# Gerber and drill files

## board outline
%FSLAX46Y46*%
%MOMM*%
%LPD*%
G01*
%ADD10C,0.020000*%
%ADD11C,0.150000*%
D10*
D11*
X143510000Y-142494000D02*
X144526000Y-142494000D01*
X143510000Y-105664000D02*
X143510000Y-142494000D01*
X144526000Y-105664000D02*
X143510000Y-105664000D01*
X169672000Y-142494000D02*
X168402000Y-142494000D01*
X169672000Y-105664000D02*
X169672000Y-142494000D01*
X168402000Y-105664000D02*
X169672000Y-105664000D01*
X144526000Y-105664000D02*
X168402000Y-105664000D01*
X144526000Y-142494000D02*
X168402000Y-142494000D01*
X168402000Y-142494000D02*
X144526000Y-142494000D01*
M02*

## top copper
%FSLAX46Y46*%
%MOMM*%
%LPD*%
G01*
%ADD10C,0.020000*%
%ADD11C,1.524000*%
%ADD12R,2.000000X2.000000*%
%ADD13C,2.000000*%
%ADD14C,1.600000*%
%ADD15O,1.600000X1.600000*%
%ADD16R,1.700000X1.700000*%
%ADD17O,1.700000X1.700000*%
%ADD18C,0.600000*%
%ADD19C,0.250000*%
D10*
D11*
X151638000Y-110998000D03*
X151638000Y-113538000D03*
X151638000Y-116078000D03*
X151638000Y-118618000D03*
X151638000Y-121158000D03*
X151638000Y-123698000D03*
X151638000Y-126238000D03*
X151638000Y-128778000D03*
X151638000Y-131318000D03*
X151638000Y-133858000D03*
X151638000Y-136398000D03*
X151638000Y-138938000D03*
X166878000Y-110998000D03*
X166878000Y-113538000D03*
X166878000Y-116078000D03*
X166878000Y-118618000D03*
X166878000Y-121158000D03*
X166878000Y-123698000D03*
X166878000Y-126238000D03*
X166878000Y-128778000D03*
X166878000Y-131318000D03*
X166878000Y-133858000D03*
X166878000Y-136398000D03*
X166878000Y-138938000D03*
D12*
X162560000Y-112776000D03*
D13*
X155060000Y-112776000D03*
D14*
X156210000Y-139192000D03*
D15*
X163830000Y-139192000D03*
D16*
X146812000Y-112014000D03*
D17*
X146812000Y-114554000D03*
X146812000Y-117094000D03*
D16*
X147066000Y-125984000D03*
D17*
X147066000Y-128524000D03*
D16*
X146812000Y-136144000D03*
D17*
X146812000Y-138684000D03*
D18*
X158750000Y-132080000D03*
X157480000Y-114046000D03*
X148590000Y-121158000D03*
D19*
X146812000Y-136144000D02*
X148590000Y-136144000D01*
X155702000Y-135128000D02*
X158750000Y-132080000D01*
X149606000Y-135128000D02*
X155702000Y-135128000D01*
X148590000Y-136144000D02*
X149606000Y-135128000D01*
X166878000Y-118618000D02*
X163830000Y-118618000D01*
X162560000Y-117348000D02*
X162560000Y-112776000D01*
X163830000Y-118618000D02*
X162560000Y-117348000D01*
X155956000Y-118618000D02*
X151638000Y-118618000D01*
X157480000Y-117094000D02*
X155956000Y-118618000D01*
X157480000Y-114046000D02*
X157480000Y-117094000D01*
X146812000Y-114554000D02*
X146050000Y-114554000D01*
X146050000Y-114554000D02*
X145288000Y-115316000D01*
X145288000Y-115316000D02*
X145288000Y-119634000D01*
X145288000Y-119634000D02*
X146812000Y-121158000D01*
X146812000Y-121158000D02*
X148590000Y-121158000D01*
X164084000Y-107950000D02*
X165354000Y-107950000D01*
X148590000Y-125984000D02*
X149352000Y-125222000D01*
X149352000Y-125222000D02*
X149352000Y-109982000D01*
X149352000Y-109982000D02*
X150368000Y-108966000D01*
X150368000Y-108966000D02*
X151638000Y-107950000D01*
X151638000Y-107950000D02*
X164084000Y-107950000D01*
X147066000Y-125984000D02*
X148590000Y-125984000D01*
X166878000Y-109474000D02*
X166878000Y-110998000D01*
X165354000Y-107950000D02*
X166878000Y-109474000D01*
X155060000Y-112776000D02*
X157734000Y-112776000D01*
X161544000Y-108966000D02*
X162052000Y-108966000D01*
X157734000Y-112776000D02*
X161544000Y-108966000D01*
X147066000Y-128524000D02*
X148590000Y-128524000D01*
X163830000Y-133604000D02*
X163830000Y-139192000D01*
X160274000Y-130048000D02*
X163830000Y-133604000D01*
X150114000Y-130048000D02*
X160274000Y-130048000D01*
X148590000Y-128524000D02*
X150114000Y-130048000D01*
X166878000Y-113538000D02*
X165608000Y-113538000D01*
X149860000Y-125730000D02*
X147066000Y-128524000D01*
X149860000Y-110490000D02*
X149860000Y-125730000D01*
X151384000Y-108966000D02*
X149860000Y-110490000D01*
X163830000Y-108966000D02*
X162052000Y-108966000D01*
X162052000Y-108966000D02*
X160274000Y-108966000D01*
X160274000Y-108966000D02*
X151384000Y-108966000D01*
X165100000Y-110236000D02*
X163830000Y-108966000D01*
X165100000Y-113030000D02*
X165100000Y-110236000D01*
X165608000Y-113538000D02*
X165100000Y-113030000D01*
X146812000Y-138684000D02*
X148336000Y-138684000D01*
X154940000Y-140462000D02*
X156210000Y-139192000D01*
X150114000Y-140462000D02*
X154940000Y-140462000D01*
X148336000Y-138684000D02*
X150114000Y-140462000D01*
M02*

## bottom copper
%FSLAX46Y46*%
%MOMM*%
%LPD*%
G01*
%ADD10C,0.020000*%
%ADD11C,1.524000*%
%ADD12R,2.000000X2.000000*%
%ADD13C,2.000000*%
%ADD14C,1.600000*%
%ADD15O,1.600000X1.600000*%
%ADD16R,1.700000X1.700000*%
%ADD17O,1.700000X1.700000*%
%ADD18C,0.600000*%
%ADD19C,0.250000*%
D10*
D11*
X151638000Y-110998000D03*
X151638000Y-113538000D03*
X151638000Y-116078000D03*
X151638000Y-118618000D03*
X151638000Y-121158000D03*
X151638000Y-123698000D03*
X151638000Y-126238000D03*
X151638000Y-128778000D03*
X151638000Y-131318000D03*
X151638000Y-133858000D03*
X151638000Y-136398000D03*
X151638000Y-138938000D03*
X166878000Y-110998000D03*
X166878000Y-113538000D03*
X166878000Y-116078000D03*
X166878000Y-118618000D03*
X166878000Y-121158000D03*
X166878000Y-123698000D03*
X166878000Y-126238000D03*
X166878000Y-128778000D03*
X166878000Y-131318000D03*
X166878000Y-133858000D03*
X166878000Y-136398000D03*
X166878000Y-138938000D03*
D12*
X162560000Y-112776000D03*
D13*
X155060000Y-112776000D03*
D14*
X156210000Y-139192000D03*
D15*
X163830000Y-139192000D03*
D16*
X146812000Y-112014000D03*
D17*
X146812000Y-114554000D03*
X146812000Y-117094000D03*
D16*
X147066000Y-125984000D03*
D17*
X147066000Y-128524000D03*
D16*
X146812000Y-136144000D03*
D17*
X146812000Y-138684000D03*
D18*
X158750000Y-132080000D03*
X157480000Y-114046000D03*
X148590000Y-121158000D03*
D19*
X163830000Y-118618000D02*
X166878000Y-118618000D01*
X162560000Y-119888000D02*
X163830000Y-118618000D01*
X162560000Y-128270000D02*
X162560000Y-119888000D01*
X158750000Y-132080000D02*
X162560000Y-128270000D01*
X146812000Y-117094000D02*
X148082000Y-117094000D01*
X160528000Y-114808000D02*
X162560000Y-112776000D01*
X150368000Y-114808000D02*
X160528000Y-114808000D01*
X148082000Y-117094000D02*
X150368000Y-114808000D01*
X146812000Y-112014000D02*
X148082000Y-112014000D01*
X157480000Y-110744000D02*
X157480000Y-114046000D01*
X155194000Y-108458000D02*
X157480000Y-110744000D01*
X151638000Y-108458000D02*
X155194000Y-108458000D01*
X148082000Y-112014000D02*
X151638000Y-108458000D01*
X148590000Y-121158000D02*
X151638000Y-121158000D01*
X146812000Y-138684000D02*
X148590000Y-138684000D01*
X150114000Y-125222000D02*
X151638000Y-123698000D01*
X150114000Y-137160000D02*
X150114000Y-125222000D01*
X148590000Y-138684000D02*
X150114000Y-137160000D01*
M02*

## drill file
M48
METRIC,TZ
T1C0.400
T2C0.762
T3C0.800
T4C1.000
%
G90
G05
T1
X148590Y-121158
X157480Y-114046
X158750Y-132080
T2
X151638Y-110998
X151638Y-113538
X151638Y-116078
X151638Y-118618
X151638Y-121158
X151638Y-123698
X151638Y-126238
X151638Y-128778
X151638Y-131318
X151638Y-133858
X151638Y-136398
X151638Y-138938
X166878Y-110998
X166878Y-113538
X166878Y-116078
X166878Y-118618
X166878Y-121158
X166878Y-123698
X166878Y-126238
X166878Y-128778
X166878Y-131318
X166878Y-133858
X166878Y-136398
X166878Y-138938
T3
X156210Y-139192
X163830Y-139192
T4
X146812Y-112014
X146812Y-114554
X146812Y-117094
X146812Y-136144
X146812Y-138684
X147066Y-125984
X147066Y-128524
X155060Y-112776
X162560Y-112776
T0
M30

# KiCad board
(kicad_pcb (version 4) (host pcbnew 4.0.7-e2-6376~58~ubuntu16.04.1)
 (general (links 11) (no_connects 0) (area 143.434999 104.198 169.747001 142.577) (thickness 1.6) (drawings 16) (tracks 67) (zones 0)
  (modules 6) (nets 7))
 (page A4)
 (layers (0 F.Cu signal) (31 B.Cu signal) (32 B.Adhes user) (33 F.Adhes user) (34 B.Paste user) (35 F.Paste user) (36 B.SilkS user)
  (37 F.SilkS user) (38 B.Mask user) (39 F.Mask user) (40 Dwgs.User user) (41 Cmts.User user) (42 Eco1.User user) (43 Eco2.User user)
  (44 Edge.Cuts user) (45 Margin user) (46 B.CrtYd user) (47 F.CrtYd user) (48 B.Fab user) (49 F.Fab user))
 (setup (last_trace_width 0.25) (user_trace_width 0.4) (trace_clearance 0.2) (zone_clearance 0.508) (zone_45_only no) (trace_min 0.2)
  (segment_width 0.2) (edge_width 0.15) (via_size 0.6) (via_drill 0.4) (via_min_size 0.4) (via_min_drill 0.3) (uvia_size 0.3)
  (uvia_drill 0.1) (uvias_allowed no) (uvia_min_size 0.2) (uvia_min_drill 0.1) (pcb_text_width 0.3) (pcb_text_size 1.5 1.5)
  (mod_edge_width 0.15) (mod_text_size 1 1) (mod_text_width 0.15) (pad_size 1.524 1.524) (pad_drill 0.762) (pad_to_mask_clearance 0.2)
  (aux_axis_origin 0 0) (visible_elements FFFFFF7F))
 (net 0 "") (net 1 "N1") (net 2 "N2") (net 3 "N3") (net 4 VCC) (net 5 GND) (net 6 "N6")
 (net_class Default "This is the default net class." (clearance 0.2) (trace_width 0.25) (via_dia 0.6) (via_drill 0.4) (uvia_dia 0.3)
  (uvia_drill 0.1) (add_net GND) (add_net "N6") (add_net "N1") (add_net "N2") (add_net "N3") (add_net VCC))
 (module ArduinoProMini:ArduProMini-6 (layer F.Cu) (at 149.098 104.648)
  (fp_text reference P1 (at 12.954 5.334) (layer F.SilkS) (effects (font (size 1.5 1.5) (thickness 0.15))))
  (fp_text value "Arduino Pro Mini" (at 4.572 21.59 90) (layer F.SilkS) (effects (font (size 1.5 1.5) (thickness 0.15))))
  (pad 7 thru_hole circle (at 2.54 6.35) (size 1.524 1.524) (drill 0.762) (layers *.Cu *.Mask F.SilkS))
  (pad 8 thru_hole circle (at 2.54 8.89) (size 1.524 1.524) (drill 0.762) (layers *.Cu *.Mask F.SilkS))
  (pad 9 thru_hole circle (at 2.54 11.43) (size 1.524 1.524) (drill 0.762) (layers *.Cu *.Mask F.SilkS))
  (pad 10 thru_hole circle (at 2.54 13.97) (size 1.524 1.524) (drill 0.762) (layers *.Cu *.Mask F.SilkS) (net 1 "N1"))
  (pad 11 thru_hole circle (at 2.54 16.51) (size 1.524 1.524) (drill 0.762) (layers *.Cu *.Mask F.SilkS) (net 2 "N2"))
  (pad 12 thru_hole circle (at 2.54 19.05) (size 1.524 1.524) (drill 0.762) (layers *.Cu *.Mask F.SilkS) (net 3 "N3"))
  (pad 13 thru_hole circle (at 2.54 21.59) (size 1.524 1.524) (drill 0.762) (layers *.Cu *.Mask F.SilkS))
  (pad 14 thru_hole circle (at 2.54 24.13) (size 1.524 1.524) (drill 0.762) (layers *.Cu *.Mask F.SilkS))
  (pad 15 thru_hole circle (at 2.54 26.67) (size 1.524 1.524) (drill 0.762) (layers *.Cu *.Mask F.SilkS))
  (pad 16 thru_hole circle (at 2.54 29.21) (size 1.524 1.524) (drill 0.762) (layers *.Cu *.Mask F.SilkS))
  (pad 17 thru_hole circle (at 2.54 31.75) (size 1.524 1.524) (drill 0.762) (layers *.Cu *.Mask F.SilkS))
  (pad 18 thru_hole circle (at 2.54 34.29) (size 1.524 1.524) (drill 0.762) (layers *.Cu *.Mask F.SilkS))
  (pad 19 thru_hole circle (at 17.78 6.35) (size 1.524 1.524) (drill 0.762) (layers *.Cu *.Mask F.SilkS) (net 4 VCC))
  (pad 20 thru_hole circle (at 17.78 8.89) (size 1.524 1.524) (drill 0.762) (layers *.Cu *.Mask F.SilkS) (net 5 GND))
  (pad 21 thru_hole circle (at 17.78 11.43) (size 1.524 1.524) (drill 0.762) (layers *.Cu *.Mask F.SilkS))
  (pad 22 thru_hole circle (at 17.78 13.97) (size 1.524 1.524) (drill 0.762) (layers *.Cu *.Mask F.SilkS) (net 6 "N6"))
  (pad 23 thru_hole circle (at 17.78 16.51) (size 1.524 1.524) (drill 0.762) (layers *.Cu *.Mask F.SilkS))
  (pad 24 thru_hole circle (at 17.78 19.05) (size 1.524 1.524) (drill 0.762) (layers *.Cu *.Mask F.SilkS))
  (pad 25 thru_hole circle (at 17.78 21.59) (size 1.524 1.524) (drill 0.762) (layers *.Cu *.Mask F.SilkS))
  (pad 26 thru_hole circle (at 17.78 24.13) (size 1.524 1.524) (drill 0.762) (layers *.Cu *.Mask F.SilkS))
  (pad 27 thru_hole circle (at 17.78 26.67) (size 1.524 1.524) (drill 0.762) (layers *.Cu *.Mask F.SilkS))
  (pad 28 thru_hole circle (at 17.78 29.21) (size 1.524 1.524) (drill 0.762) (layers *.Cu *.Mask F.SilkS))
  (pad 29 thru_hole circle (at 17.78 31.75) (size 1.524 1.524) (drill 0.762) (layers *.Cu *.Mask F.SilkS))
  (pad 30 thru_hole circle (at 17.78 34.29) (size 1.524 1.524) (drill 0.762) (layers *.Cu *.Mask F.SilkS)))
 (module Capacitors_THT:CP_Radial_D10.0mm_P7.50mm (layer F.Cu) (at 162.56 112.776 180)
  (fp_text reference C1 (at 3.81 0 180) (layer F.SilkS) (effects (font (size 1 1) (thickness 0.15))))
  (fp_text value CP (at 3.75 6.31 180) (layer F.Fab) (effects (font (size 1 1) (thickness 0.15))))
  (pad 1 thru_hole rect (at 0 0 180) (size 2 2) (drill 1) (layers *.Cu *.Mask) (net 6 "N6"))
  (pad 2 thru_hole circle (at 7.5 0 180) (size 2 2) (drill 1) (layers *.Cu *.Mask) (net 5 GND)))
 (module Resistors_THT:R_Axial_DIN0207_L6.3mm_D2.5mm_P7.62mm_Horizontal (layer F.Cu) (at 156.21 139.192)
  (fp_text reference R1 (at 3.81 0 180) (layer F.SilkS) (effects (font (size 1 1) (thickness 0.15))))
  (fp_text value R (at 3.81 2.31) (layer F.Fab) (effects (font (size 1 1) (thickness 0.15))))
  (pad 1 thru_hole circle (at 0 0) (size 1.6 1.6) (drill 0.8) (layers *.Cu *.Mask) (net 3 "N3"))
  (pad 2 thru_hole oval (at 7.62 0) (size 1.6 1.6) (drill 0.8) (layers *.Cu *.Mask) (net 5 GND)))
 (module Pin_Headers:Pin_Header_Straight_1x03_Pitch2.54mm (layer F.Cu) (at 146.812 112.014)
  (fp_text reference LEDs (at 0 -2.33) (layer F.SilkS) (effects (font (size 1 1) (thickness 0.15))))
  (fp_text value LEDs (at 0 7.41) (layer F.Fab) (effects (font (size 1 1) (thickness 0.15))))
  (pad 1 thru_hole rect (at 0 0) (size 1.7 1.7) (drill 1) (layers *.Cu *.Mask) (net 1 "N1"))
  (pad 2 thru_hole oval (at 0 2.54) (size 1.7 1.7) (drill 1) (layers *.Cu *.Mask) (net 2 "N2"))
  (pad 3 thru_hole oval (at 0 5.08) (size 1.7 1.7) (drill 1) (layers *.Cu *.Mask) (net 6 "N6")))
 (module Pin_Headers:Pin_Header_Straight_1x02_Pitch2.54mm (layer F.Cu) (at 147.066 125.984)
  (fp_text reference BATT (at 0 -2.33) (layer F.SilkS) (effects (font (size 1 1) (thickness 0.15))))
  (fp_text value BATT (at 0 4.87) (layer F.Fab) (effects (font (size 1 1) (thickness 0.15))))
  (pad 1 thru_hole rect (at 0 0) (size 1.7 1.7) (drill 1) (layers *.Cu *.Mask) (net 4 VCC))
  (pad 2 thru_hole oval (at 0 2.54) (size 1.7 1.7) (drill 1) (layers *.Cu *.Mask) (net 5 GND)))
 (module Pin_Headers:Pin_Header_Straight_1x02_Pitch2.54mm (layer F.Cu) (at 146.812 136.144)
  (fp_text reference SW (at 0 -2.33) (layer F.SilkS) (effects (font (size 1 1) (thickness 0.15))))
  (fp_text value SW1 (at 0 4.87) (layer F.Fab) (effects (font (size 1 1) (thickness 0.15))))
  (pad 1 thru_hole rect (at 0 0) (size 1.7 1.7) (drill 1) (layers *.Cu *.Mask) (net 6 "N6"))
  (pad 2 thru_hole oval (at 0 2.54) (size 1.7 1.7) (drill 1) (layers *.Cu *.Mask) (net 3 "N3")))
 (gr_line (start 143.51 142.494) (end 144.526 142.494) (angle 90) (layer Edge.Cuts) (width 0.15))
 (gr_line (start 143.51 105.664) (end 143.51 142.494) (angle 90) (layer Edge.Cuts) (width 0.15))
 (gr_line (start 144.526 105.664) (end 143.51 105.664) (angle 90) (layer Edge.Cuts) (width 0.15))
 (gr_line (start 169.672 142.494) (end 168.402 142.494) (angle 90) (layer Edge.Cuts) (width 0.15))
 (gr_line (start 169.672 105.664) (end 169.672 142.494) (angle 90) (layer Edge.Cuts) (width 0.15))
 (gr_line (start 168.402 105.664) (end 169.672 105.664) (angle 90) (layer Edge.Cuts) (width 0.15))
 (gr_line (start 144.526 105.664) (end 168.402 105.664) (angle 90) (layer Edge.Cuts) (width 0.15))
 (gr_line (start 144.526 142.494) (end 168.402 142.494) (angle 90) (layer Edge.Cuts) (width 0.15))
 (gr_line (start 168.402 142.494) (end 144.526 142.494) (angle 90) (layer Edge.Cuts) (width 0.15))
 (segment (start 146.812 136.144) (end 148.59 136.144) (width 0.25) (layer F.Cu) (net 6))
 (segment (start 163.83 118.618) (end 166.878 118.618) (width 0.25) (layer B.Cu) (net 6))
 (segment (start 162.56 119.888) (end 163.83 118.618) (width 0.25) (layer B.Cu) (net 6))
 (segment (start 162.56 128.27) (end 162.56 119.888) (width 0.25) (layer B.Cu) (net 6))
 (segment (start 158.75 132.08) (end 162.56 128.27) (width 0.25) (layer B.Cu) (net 6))
 (via (at 158.75 132.08) (size 0.6) (drill 0.4) (layers F.Cu B.Cu) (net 6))
 (segment (start 155.702 135.128) (end 158.75 132.08) (width 0.25) (layer F.Cu) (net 6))
 (segment (start 149.606 135.128) (end 155.702 135.128) (width 0.25) (layer F.Cu) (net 6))
 (segment (start 148.59 136.144) (end 149.606 135.128) (width 0.25) (layer F.Cu) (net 6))
 (segment (start 146.812 117.094) (end 148.082 117.094) (width 0.25) (layer B.Cu) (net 6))
 (segment (start 160.528 114.808) (end 162.56 112.776) (width 0.25) (layer B.Cu) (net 6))
 (segment (start 150.368 114.808) (end 160.528 114.808) (width 0.25) (layer B.Cu) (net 6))
 (segment (start 148.082 117.094) (end 150.368 114.808) (width 0.25) (layer B.Cu) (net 6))
 (segment (start 166.878 118.618) (end 163.83 118.618) (width 0.25) (layer F.Cu) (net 6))
 (segment (start 162.56 117.348) (end 162.56 112.776) (width 0.25) (layer F.Cu) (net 6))
 (segment (start 163.83 118.618) (end 162.56 117.348) (width 0.25) (layer F.Cu) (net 6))
 (segment (start 146.812 112.014) (end 148.082 112.014) (width 0.25) (layer B.Cu) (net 1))
 (segment (start 155.956 118.618) (end 151.638 118.618) (width 0.25) (layer F.Cu) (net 1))
 (segment (start 157.48 117.094) (end 155.956 118.618) (width 0.25) (layer F.Cu) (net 1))
 (segment (start 157.48 114.046) (end 157.48 117.094) (width 0.25) (layer F.Cu) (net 1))
 (via (at 157.48 114.046) (size 0.6) (drill 0.4) (layers F.Cu B.Cu) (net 1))
 (segment (start 157.48 110.744) (end 157.48 114.046) (width 0.25) (layer B.Cu) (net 1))
 (segment (start 155.194 108.458) (end 157.48 110.744) (width 0.25) (layer B.Cu) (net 1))
 (segment (start 151.638 108.458) (end 155.194 108.458) (width 0.25) (layer B.Cu) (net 1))
 (segment (start 148.082 112.014) (end 151.638 108.458) (width 0.25) (layer B.Cu) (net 1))
 (segment (start 146.812 114.554) (end 146.05 114.554) (width 0.25) (layer F.Cu) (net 2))
 (segment (start 146.05 114.554) (end 145.288 115.316) (width 0.25) (layer F.Cu) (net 2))
 (segment (start 145.288 115.316) (end 145.288 119.634) (width 0.25) (layer F.Cu) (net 2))
 (segment (start 145.288 119.634) (end 146.812 121.158) (width 0.25) (layer F.Cu) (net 2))
 (segment (start 146.812 121.158) (end 148.59 121.158) (width 0.25) (layer F.Cu) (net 2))
 (via (at 148.59 121.158) (size 0.6) (drill 0.4) (layers F.Cu B.Cu) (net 2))
 (segment (start 148.59 121.158) (end 151.638 121.158) (width 0.25) (layer B.Cu) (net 2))
 (segment (start 164.084 107.95) (end 165.354 107.95) (width 0.25) (layer F.Cu) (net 4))
 (segment (start 148.59 125.984) (end 149.352 125.222) (width 0.25) (layer F.Cu) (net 4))
 (segment (start 149.352 125.222) (end 149.352 109.982) (width 0.25) (layer F.Cu) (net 4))
 (segment (start 149.352 109.982) (end 150.368 108.966) (width 0.25) (layer F.Cu) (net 4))
 (segment (start 150.368 108.966) (end 151.638 107.95) (width 0.25) (layer F.Cu) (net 4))
 (segment (start 151.638 107.95) (end 164.084 107.95) (width 0.25) (layer F.Cu) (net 4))
 (segment (start 147.066 125.984) (end 148.59 125.984) (width 0.25) (layer F.Cu) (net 4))
 (segment (start 166.878 109.474) (end 166.878 110.998) (width 0.25) (layer F.Cu) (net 4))
 (segment (start 165.354 107.95) (end 166.878 109.474) (width 0.25) (layer F.Cu) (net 4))
 (segment (start 155.06 112.776) (end 157.734 112.776) (width 0.25) (layer F.Cu) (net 5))
 (segment (start 161.544 108.966) (end 162.052 108.966) (width 0.25) (layer F.Cu) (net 5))
 (segment (start 157.734 112.776) (end 161.544 108.966) (width 0.25) (layer F.Cu) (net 5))
 (segment (start 147.066 128.524) (end 148.59 128.524) (width 0.25) (layer F.Cu) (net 5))
 (segment (start 163.83 133.604) (end 163.83 139.192) (width 0.25) (layer F.Cu) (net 5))
 (segment (start 160.274 130.048) (end 163.83 133.604) (width 0.25) (layer F.Cu) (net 5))
 (segment (start 150.114 130.048) (end 160.274 130.048) (width 0.25) (layer F.Cu) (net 5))
 (segment (start 148.59 128.524) (end 150.114 130.048) (width 0.25) (layer F.Cu) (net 5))
 (segment (start 166.878 113.538) (end 165.608 113.538) (width 0.25) (layer F.Cu) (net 5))
 (segment (start 149.86 125.73) (end 147.066 128.524) (width 0.25) (layer F.Cu) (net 5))
 (segment (start 149.86 110.49) (end 149.86 125.73) (width 0.25) (layer F.Cu) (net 5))
 (segment (start 151.384 108.966) (end 149.86 110.49) (width 0.25) (layer F.Cu) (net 5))
 (segment (start 163.83 108.966) (end 162.052 108.966) (width 0.25) (layer F.Cu) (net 5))
 (segment (start 162.052 108.966) (end 160.274 108.966) (width 0.25) (layer F.Cu) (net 5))
 (segment (start 160.274 108.966) (end 151.384 108.966) (width 0.25) (layer F.Cu) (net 5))
 (segment (start 165.1 110.236) (end 163.83 108.966) (width 0.25) (layer F.Cu) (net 5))
 (segment (start 165.1 113.03) (end 165.1 110.236) (width 0.25) (layer F.Cu) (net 5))
 (segment (start 165.608 113.538) (end 165.1 113.03) (width 0.25) (layer F.Cu) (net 5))
 (segment (start 146.812 138.684) (end 148.59 138.684) (width 0.25) (layer B.Cu) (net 3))
 (segment (start 150.114 125.222) (end 151.638 123.698) (width 0.25) (layer B.Cu) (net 3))
 (segment (start 150.114 137.16) (end 150.114 125.222) (width 0.25) (layer B.Cu) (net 3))
 (segment (start 148.59 138.684) (end 150.114 137.16) (width 0.25) (layer B.Cu) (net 3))
 (segment (start 146.812 138.684) (end 148.336 138.684) (width 0.25) (layer F.Cu) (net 3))
 (segment (start 154.94 140.462) (end 156.21 139.192) (width 0.25) (layer F.Cu) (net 3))
 (segment (start 150.114 140.462) (end 154.94 140.462) (width 0.25) (layer F.Cu) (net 3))
 (segment (start 148.336 138.684) (end 150.114 140.462) (width 0.25) (layer F.Cu) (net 3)))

